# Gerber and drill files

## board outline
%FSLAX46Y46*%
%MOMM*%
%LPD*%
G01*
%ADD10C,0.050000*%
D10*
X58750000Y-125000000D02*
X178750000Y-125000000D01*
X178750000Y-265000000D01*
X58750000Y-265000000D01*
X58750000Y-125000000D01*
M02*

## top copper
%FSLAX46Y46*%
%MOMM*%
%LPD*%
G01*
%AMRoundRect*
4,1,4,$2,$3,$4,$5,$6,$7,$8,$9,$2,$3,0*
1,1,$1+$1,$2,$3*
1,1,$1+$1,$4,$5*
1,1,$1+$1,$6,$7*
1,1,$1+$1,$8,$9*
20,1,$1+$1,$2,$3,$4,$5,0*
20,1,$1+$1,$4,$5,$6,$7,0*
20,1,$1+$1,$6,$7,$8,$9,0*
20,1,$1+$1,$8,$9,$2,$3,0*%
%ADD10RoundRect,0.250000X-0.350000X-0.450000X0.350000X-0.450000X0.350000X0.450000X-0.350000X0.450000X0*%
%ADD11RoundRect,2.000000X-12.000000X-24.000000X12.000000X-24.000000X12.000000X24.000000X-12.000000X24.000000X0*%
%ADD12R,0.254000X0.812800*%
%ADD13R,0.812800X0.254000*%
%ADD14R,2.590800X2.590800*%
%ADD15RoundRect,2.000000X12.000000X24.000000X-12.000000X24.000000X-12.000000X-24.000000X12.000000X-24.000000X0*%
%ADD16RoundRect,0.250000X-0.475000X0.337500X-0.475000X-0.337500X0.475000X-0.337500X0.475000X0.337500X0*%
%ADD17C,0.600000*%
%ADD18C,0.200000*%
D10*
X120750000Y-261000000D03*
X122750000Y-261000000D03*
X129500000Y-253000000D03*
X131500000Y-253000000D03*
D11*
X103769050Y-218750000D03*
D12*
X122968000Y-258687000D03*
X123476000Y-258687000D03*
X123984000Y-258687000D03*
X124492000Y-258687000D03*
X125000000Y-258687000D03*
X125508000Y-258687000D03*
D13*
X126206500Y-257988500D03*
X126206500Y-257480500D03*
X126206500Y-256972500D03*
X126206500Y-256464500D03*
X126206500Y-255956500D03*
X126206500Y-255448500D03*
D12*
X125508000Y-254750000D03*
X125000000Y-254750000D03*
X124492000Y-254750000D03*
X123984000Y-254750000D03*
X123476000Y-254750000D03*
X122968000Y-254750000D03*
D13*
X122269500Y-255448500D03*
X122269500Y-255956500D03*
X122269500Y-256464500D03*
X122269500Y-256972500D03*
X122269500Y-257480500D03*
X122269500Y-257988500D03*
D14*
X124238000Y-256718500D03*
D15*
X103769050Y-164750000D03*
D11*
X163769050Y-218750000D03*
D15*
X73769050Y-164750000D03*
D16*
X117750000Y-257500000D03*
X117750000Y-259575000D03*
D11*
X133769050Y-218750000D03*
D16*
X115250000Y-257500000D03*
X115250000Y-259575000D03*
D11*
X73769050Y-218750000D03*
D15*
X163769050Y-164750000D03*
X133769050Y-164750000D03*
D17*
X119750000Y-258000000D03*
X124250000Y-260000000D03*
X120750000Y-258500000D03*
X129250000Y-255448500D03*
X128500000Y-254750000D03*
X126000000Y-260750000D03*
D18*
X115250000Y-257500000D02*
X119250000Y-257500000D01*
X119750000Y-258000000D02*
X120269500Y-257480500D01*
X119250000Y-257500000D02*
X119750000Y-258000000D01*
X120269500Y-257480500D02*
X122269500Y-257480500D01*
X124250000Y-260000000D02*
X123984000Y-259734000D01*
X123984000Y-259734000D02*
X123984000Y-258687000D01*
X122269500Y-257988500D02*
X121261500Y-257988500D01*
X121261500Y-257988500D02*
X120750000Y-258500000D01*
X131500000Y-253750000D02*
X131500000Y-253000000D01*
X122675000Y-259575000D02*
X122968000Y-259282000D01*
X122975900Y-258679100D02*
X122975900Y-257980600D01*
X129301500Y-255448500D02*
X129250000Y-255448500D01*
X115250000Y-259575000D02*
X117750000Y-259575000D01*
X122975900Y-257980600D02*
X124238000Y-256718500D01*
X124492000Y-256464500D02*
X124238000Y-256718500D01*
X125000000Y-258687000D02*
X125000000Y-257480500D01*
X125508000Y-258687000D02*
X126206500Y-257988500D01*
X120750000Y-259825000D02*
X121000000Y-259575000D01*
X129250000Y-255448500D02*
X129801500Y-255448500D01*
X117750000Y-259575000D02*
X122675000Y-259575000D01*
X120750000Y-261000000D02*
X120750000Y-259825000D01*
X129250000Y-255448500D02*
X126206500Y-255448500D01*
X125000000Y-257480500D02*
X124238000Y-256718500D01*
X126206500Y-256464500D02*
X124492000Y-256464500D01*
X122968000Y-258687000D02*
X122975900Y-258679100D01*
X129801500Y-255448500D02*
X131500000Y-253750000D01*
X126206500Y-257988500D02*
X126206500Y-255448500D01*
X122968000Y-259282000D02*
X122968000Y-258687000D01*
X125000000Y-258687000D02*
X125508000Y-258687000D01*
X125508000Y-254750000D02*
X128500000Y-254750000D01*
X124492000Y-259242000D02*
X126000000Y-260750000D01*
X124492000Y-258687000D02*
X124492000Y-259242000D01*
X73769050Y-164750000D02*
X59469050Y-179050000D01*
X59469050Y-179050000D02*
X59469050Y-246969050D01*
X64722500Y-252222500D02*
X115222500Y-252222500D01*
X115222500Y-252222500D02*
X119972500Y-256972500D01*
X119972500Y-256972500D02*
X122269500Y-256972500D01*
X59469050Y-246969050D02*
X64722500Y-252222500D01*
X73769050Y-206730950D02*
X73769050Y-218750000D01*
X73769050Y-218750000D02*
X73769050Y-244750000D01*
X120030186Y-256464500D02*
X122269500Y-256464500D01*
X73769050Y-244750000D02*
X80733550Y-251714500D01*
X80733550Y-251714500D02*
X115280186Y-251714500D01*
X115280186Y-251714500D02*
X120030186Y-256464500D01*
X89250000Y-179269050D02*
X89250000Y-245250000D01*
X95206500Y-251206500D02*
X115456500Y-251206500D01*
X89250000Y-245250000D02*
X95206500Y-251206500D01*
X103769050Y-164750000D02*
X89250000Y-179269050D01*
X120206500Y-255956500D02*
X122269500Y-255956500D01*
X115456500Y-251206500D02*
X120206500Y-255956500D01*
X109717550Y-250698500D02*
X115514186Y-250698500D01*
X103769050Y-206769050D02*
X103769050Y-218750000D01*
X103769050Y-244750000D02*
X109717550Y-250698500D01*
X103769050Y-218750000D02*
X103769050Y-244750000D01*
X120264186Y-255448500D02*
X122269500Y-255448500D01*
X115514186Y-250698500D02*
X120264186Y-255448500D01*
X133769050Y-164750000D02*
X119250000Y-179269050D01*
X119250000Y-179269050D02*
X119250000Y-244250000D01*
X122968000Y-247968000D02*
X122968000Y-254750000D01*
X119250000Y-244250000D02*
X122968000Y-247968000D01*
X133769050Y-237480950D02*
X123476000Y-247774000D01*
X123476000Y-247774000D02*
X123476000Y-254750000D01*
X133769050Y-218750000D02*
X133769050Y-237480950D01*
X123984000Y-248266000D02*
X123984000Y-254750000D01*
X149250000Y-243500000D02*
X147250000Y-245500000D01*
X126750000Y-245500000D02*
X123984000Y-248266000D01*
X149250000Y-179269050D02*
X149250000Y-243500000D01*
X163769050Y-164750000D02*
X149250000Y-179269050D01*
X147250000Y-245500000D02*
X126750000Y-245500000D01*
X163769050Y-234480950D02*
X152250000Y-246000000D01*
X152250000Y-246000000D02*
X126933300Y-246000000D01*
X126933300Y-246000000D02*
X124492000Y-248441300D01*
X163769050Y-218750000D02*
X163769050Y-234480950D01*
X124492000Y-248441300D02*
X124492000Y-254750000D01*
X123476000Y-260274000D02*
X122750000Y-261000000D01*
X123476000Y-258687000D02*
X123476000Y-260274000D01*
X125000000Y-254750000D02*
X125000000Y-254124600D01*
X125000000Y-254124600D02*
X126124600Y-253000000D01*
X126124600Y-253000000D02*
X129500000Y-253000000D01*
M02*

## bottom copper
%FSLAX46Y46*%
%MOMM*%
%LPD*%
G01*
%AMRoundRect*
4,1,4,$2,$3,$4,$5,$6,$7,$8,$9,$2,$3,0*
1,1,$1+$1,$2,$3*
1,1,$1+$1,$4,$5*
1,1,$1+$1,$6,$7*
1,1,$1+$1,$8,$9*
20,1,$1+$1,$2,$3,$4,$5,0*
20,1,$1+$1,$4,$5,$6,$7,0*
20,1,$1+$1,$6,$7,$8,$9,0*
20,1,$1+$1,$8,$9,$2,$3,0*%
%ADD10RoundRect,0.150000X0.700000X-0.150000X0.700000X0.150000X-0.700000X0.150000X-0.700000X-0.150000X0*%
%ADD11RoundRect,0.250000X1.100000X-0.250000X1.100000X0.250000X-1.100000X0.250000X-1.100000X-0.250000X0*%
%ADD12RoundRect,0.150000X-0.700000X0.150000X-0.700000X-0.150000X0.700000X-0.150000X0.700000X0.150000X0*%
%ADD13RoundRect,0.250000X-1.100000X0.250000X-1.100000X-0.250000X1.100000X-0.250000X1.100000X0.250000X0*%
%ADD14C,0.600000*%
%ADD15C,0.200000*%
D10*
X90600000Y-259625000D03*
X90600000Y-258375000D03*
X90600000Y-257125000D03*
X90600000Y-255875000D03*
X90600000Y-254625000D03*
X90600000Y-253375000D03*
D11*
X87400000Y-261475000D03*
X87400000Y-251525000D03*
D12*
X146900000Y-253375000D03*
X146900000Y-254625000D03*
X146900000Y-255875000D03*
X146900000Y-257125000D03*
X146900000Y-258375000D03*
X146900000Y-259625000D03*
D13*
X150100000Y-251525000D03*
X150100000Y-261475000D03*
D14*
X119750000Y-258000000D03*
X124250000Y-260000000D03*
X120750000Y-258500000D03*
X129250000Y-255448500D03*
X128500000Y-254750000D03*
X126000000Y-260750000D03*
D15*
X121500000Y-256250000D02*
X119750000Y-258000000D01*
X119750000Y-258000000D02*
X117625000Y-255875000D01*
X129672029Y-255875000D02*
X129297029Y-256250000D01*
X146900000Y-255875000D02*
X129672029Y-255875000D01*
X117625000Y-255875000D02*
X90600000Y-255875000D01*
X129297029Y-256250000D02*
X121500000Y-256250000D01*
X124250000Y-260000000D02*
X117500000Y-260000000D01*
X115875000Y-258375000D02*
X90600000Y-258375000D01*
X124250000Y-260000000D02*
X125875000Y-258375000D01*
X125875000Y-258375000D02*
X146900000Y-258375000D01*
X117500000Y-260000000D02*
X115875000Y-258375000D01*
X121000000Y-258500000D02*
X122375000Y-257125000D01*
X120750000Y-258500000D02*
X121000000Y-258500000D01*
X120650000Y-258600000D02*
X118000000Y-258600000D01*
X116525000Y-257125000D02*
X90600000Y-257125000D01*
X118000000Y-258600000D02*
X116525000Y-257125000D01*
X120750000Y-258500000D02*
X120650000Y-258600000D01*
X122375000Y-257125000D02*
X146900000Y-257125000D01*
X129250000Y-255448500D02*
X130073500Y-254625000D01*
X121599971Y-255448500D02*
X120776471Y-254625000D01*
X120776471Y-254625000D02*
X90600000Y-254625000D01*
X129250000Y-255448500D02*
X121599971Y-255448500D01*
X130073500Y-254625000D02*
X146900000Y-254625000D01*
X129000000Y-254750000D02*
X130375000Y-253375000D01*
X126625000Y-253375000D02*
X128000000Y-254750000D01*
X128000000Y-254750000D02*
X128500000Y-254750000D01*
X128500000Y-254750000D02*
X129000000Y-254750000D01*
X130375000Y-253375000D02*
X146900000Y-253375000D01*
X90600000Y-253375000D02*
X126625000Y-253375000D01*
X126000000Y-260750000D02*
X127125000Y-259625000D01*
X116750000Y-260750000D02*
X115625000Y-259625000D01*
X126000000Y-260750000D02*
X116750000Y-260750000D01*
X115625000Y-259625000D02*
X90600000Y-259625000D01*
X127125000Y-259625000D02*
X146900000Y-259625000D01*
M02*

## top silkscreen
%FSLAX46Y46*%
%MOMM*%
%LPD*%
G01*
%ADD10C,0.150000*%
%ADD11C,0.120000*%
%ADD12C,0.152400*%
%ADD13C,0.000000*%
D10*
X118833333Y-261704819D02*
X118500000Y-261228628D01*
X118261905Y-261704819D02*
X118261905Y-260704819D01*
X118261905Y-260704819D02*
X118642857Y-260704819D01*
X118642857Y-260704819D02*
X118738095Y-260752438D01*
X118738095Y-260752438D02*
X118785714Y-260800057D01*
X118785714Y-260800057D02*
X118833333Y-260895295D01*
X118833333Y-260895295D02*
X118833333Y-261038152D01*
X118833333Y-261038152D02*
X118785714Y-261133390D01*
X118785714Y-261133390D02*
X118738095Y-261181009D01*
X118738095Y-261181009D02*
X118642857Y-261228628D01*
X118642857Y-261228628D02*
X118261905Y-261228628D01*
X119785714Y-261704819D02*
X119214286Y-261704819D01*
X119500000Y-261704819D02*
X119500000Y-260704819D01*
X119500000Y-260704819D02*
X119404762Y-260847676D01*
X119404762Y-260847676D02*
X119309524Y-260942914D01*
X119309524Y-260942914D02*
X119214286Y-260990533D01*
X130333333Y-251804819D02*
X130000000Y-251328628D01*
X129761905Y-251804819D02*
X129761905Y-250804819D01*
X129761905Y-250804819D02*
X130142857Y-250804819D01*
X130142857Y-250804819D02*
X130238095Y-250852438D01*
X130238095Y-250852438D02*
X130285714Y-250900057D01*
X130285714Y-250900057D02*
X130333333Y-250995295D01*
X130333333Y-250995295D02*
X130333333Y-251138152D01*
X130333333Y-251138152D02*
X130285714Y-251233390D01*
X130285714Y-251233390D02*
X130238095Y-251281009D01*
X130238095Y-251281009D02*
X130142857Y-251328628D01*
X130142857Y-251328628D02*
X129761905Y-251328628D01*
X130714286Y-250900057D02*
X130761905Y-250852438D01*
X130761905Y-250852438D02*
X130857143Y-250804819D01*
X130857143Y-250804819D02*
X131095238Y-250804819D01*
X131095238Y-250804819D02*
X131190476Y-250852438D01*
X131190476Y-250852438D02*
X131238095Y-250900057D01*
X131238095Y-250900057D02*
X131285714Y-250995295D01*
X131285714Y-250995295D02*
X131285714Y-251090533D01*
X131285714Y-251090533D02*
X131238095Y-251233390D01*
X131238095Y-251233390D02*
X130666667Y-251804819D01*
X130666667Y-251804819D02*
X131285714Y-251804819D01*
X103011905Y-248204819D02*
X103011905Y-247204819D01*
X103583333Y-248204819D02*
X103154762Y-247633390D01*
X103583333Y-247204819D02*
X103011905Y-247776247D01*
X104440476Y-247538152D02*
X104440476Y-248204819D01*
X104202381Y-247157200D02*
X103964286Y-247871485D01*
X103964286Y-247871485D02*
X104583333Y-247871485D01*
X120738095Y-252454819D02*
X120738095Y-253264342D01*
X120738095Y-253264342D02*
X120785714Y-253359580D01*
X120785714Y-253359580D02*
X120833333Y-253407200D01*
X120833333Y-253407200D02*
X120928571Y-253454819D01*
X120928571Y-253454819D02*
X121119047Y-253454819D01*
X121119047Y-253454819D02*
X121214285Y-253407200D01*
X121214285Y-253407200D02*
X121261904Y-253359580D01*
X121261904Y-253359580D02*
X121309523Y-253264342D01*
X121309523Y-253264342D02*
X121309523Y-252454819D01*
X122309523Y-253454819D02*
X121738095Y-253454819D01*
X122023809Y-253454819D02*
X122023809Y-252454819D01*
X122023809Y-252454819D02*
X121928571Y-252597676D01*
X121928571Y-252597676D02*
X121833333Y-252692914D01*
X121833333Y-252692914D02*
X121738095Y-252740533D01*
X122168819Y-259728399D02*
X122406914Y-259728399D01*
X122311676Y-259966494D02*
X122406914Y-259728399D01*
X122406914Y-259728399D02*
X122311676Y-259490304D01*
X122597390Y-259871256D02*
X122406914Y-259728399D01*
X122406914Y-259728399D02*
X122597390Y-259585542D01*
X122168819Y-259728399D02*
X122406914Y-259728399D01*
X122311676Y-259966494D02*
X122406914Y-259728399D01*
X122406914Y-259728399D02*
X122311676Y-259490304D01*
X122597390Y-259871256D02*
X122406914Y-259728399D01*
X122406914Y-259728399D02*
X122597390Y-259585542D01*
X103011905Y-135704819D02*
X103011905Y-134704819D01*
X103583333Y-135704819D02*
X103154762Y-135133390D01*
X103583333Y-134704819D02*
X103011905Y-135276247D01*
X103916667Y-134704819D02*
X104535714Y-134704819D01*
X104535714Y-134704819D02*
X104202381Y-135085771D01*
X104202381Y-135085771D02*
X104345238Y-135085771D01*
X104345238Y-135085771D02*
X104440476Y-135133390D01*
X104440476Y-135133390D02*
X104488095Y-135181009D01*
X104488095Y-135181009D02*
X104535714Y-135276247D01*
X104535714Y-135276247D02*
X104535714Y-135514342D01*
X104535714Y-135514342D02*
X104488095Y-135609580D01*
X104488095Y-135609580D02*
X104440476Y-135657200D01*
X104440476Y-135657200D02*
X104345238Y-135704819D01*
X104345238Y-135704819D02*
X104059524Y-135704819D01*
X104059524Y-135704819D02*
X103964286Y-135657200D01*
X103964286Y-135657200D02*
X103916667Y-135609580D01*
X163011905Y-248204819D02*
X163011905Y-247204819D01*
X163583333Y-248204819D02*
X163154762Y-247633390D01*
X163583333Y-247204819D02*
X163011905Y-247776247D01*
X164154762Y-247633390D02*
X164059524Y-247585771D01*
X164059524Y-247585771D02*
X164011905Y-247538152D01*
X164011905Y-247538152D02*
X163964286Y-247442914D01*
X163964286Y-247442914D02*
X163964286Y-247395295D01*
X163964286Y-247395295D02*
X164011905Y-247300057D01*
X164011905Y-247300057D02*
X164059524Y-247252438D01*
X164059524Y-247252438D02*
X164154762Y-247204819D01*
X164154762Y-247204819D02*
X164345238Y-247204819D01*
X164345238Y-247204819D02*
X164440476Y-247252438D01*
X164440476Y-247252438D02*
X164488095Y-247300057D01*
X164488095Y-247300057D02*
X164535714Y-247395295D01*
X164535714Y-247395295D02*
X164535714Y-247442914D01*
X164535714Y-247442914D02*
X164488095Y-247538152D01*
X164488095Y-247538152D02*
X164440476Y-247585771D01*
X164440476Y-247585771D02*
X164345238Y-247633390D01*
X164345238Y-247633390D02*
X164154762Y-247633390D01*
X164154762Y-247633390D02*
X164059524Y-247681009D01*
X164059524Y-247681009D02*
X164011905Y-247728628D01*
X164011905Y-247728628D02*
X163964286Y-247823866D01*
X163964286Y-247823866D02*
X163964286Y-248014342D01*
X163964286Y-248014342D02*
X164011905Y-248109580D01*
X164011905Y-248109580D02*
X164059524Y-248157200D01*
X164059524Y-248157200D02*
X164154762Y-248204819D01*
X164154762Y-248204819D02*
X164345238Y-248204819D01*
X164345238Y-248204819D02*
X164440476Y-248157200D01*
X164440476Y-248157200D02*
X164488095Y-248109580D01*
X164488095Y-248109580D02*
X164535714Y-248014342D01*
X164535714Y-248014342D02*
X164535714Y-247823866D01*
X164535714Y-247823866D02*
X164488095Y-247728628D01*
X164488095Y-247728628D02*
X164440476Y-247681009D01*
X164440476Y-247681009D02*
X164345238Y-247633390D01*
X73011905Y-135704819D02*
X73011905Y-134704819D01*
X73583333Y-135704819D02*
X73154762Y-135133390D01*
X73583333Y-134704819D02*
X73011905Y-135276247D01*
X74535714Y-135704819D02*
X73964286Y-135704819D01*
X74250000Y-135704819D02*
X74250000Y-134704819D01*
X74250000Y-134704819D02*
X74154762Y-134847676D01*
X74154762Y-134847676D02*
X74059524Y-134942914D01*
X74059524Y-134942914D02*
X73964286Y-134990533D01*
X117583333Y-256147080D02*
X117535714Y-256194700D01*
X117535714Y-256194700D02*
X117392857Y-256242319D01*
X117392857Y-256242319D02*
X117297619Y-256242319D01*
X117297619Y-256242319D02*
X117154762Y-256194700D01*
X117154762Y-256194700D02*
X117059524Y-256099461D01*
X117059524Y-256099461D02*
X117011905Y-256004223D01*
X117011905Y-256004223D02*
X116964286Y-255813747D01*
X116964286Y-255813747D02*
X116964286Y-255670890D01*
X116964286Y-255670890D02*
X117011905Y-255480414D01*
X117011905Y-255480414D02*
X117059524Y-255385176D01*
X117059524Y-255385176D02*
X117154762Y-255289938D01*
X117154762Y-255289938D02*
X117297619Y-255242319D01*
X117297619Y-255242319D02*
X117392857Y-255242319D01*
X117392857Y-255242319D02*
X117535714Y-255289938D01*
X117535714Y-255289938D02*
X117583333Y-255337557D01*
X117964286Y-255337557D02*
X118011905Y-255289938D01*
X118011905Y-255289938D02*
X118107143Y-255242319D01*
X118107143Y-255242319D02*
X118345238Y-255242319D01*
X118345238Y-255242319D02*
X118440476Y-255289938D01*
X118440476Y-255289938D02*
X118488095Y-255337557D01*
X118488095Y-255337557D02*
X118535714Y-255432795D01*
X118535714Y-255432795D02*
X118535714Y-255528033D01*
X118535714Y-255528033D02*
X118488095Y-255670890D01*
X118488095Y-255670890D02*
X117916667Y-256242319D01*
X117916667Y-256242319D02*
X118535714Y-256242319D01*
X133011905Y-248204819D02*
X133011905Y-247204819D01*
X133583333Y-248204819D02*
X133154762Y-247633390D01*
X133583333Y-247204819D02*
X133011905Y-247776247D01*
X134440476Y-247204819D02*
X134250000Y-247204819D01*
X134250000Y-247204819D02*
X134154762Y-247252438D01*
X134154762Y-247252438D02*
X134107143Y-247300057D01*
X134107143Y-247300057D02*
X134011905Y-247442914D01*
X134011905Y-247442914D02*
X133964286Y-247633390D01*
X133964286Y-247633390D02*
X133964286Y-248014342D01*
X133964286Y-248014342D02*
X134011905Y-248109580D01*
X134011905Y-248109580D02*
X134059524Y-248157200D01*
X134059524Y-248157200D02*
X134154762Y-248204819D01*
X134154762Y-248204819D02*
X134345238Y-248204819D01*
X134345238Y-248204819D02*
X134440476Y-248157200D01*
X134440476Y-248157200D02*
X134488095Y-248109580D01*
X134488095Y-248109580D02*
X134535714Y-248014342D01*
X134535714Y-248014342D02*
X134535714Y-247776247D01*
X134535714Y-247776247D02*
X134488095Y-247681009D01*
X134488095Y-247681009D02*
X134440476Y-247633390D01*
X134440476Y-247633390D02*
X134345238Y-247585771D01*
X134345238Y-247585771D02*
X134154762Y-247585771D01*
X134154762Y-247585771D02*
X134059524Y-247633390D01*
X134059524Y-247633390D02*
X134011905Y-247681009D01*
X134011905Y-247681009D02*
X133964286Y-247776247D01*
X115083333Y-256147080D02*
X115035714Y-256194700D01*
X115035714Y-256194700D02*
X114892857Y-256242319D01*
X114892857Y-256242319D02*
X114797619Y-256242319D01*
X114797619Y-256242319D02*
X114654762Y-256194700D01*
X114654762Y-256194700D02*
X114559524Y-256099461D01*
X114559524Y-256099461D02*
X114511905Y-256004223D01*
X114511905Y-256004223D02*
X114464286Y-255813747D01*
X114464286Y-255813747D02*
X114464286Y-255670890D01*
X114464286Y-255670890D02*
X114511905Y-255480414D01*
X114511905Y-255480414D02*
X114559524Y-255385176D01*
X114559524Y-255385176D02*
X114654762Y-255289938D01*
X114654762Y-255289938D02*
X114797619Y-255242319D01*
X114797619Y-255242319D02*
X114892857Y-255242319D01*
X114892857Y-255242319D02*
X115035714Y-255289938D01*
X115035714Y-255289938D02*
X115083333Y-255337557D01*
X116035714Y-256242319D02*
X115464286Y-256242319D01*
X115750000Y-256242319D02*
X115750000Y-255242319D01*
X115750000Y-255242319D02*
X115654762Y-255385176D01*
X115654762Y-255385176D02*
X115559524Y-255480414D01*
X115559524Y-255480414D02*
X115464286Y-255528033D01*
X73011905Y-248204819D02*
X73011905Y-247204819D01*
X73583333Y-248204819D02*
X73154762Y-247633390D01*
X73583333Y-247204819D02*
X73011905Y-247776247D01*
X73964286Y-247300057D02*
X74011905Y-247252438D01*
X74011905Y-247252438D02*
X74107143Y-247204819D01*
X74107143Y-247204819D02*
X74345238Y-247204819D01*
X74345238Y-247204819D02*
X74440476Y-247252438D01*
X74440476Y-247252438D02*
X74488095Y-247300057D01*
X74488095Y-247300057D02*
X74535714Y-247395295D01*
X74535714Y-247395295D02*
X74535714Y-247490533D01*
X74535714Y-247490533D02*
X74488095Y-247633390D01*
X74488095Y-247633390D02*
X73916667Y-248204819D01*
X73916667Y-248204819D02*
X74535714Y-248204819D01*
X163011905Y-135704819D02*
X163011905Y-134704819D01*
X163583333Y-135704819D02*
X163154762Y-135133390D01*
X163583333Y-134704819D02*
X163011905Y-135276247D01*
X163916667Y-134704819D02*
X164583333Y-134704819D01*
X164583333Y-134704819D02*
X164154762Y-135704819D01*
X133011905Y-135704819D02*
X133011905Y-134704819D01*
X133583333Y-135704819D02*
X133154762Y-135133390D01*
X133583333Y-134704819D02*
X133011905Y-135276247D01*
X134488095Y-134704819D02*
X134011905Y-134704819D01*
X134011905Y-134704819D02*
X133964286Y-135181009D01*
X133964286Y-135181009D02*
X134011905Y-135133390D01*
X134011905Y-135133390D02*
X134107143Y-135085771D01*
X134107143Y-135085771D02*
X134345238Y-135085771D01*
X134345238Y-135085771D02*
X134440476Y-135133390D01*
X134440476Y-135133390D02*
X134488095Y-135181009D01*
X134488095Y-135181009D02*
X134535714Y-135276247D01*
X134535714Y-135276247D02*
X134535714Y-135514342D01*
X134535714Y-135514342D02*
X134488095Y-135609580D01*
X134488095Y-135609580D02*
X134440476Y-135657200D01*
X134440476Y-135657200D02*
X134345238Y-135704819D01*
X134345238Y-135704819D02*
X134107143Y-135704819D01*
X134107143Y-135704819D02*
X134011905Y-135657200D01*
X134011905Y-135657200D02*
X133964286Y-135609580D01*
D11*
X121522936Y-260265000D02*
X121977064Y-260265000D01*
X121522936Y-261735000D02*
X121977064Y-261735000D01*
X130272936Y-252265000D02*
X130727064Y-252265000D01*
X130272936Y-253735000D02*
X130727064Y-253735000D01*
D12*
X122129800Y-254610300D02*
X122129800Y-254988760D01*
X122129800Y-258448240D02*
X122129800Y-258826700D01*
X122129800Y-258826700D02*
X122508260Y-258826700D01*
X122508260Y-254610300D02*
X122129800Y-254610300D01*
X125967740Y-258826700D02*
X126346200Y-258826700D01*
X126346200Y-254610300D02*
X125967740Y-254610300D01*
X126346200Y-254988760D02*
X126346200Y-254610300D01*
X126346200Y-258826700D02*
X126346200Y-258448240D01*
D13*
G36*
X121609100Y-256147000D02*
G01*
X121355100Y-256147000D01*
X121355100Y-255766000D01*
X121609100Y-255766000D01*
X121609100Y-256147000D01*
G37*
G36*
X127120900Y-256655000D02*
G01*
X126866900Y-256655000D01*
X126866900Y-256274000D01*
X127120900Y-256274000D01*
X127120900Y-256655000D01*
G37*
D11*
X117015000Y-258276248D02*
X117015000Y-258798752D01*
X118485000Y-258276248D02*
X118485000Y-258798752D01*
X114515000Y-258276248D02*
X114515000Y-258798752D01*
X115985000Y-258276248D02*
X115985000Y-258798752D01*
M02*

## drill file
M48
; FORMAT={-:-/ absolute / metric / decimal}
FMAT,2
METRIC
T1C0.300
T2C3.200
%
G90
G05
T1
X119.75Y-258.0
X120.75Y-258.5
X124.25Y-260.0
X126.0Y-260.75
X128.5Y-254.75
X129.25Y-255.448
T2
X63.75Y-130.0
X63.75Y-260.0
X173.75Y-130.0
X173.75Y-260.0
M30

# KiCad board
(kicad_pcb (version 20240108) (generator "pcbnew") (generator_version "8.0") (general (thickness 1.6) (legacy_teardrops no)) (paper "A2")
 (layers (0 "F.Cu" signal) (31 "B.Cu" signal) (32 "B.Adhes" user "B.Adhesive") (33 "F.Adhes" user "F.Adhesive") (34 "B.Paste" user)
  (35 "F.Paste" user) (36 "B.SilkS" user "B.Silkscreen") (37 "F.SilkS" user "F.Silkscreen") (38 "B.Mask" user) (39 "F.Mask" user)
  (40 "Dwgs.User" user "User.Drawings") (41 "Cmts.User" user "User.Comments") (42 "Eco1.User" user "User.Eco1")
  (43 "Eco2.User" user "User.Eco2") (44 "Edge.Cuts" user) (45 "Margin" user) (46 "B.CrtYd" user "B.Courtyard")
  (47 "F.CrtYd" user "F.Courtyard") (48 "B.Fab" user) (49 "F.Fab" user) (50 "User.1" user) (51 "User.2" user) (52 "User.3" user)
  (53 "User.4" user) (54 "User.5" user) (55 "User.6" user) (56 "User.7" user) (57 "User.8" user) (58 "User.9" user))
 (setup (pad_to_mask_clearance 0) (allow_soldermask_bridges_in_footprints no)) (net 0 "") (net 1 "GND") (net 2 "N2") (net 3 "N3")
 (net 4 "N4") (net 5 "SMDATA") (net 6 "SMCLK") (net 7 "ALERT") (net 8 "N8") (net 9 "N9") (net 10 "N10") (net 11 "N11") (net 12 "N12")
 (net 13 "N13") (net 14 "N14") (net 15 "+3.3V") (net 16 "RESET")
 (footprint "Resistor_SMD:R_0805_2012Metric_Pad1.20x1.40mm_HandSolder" (layer "F.Cu") (at 121.75 261)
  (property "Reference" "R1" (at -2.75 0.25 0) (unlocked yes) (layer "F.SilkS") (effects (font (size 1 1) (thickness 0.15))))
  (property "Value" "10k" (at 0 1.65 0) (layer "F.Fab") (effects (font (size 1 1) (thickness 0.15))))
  (fp_line (start -0.227064 -0.735) (end 0.227064 -0.735) (stroke (width 0.12) (type solid)) (layer "F.SilkS"))
  (fp_line (start -0.227064 0.735) (end 0.227064 0.735) (stroke (width 0.12) (type solid)) (layer "F.SilkS"))
  (pad "1" smd roundrect (at -1 0) (size 1.2 1.4) (layers "F.Cu" "F.Paste" "F.Mask") (roundrect_rratio 0.208333) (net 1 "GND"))
  (pad "2" smd roundrect (at 1 0) (size 1.2 1.4) (layers "F.Cu" "F.Paste" "F.Mask") (roundrect_rratio 0.208333) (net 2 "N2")))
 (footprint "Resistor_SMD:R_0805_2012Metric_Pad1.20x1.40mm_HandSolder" (layer "F.Cu") (at 130.5 253)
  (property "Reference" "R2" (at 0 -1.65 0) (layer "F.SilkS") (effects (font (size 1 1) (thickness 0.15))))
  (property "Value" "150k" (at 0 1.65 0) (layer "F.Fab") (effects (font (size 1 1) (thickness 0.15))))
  (fp_line (start -0.227064 -0.735) (end 0.227064 -0.735) (stroke (width 0.12) (type solid)) (layer "F.SilkS"))
  (fp_line (start -0.227064 0.735) (end 0.227064 0.735) (stroke (width 0.12) (type solid)) (layer "F.SilkS"))
  (pad "1" smd roundrect (at -1 0) (size 1.2 1.4) (layers "F.Cu" "F.Paste" "F.Mask") (roundrect_rratio 0.208333) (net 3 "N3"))
  (pad "2" smd roundrect (at 1 0) (size 1.2 1.4) (layers "F.Cu" "F.Paste" "F.Mask") (roundrect_rratio 0.208333) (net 1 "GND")))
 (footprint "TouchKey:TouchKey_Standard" (layer "F.Cu") (at 103.76905 218.75)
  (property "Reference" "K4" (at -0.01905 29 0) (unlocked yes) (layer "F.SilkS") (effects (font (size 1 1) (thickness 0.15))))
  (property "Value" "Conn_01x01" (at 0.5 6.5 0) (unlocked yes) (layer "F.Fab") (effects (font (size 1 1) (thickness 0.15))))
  (pad "1" smd roundrect (at 0 0) (size 28 52) (layers "F.Cu") (roundrect_rratio 0.07142857143) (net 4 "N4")))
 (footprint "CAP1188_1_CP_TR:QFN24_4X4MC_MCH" (layer "F.Cu") (at 124.238 256.7185 90)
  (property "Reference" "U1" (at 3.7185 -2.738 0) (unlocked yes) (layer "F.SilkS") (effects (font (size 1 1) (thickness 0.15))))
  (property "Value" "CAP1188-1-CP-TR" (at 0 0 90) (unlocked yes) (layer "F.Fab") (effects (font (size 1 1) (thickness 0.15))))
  (fp_line (start 2.1082 -2.1082) (end 1.72974 -2.1082) (stroke (width 0.1524) (type solid)) (layer "F.SilkS"))
  (fp_line (start -1.72974 -2.1082) (end -2.1082 -2.1082) (stroke (width 0.1524) (type solid)) (layer "F.SilkS"))
  (fp_line (start -2.1082 -2.1082) (end -2.1082 -1.72974) (stroke (width 0.1524) (type solid)) (layer "F.SilkS"))
  (fp_line (start 2.1082 -1.72974) (end 2.1082 -2.1082) (stroke (width 0.1524) (type solid)) (layer "F.SilkS"))
  (fp_line (start -2.1082 1.72974) (end -2.1082 2.1082) (stroke (width 0.1524) (type solid)) (layer "F.SilkS"))
  (fp_line (start 2.1082 2.1082) (end 2.1082 1.72974) (stroke (width 0.1524) (type solid)) (layer "F.SilkS"))
  (fp_line (start 1.72974 2.1082) (end 2.1082 2.1082) (stroke (width 0.1524) (type solid)) (layer "F.SilkS"))
  (fp_line (start -2.1082 2.1082) (end -1.72974 2.1082) (stroke (width 0.1524) (type solid)) (layer "F.SilkS"))
  (fp_poly
   (pts (xy 0.5715 -2.6289) (xy 0.5715 -2.8829) (xy 0.9525 -2.8829) (xy 0.9525 -2.6289)) (stroke (width 0) (type solid)) (fill solid)
   (layer "F.SilkS"))
  (fp_poly
   (pts (xy 0.0635 2.6289) (xy 0.0635 2.8829) (xy 0.4445 2.8829) (xy 0.4445 2.6289)) (stroke (width 0) (type solid)) (fill solid)
   (layer "F.SilkS"))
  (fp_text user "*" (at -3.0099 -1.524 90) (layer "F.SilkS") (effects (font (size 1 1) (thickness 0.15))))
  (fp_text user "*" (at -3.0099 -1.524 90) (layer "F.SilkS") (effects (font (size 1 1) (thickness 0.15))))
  (pad "1" smd rect (at -1.9685 -1.27 180) (size 0.254 0.8128) (layers "F.Cu" "F.Paste" "F.Mask") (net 1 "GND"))
  (pad "2" smd rect (at -1.9685 -0.762 180) (size 0.254 0.8128) (layers "F.Cu" "F.Paste" "F.Mask") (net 2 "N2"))
  (pad "3" smd rect (at -1.9685 -0.254 180) (size 0.254 0.8128) (layers "F.Cu" "F.Paste" "F.Mask") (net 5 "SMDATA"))
  (pad "4" smd rect (at -1.9685 0.254 180) (size 0.254 0.8128) (layers "F.Cu" "F.Paste" "F.Mask") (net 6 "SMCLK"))
  (pad "5" smd rect (at -1.9685 0.762 180) (size 0.254 0.8128) (layers "F.Cu" "F.Paste" "F.Mask") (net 1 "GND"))
  (pad "6" smd rect (at -1.9685 1.27 180) (size 0.254 0.8128) (layers "F.Cu" "F.Paste" "F.Mask") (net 1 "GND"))
  (pad "7" smd rect (at -1.27 1.9685 90) (size 0.254 0.8128) (layers "F.Cu" "F.Paste" "F.Mask") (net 1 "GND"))
  (pad "8" smd rect (at -0.762 1.9685 90) (size 0.254 0.8128) (layers "F.Cu" "F.Paste" "F.Mask") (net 1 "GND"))
  (pad "9" smd rect (at -0.254 1.9685 90) (size 0.254 0.8128) (layers "F.Cu" "F.Paste" "F.Mask") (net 1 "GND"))
  (pad "10" smd rect (at 0.254 1.9685 90) (size 0.254 0.8128) (layers "F.Cu" "F.Paste" "F.Mask") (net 1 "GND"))
  (pad "11" smd rect (at 0.762 1.9685 90) (size 0.254 0.8128) (layers "F.Cu" "F.Paste" "F.Mask") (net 1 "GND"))
  (pad "12" smd rect (at 1.27 1.9685 90) (size 0.254 0.8128) (layers "F.Cu" "F.Paste" "F.Mask") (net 1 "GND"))
  (pad "13" smd rect (at 1.9685 1.27 180) (size 0.254 0.8128) (layers "F.Cu" "F.Paste" "F.Mask") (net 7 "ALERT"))
  (pad "14" smd rect (at 1.9685 0.762 180) (size 0.254 0.8128) (layers "F.Cu" "F.Paste" "F.Mask") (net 3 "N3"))
  (pad "15" smd rect (at 1.9685 0.254 180) (size 0.254 0.8128) (layers "F.Cu" "F.Paste" "F.Mask") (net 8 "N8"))
  (pad "16" smd rect (at 1.9685 -0.254 180) (size 0.254 0.8128) (layers "F.Cu" "F.Paste" "F.Mask") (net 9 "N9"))
  (pad "17" smd rect (at 1.9685 -0.762 180) (size 0.254 0.8128) (layers "F.Cu" "F.Paste" "F.Mask") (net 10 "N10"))
  (pad "18" smd rect (at 1.9685 -1.27 180) (size 0.254 0.8128) (layers "F.Cu" "F.Paste" "F.Mask") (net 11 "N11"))
  (pad "19" smd rect (at 1.27 -1.9685 90) (size 0.254 0.8128) (layers "F.Cu" "F.Paste" "F.Mask") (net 4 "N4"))
  (pad "20" smd rect (at 0.762 -1.9685 90) (size 0.254 0.8128) (layers "F.Cu" "F.Paste" "F.Mask") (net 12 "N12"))
  (pad "21" smd rect (at 0.254 -1.9685 90) (size 0.254 0.8128) (layers "F.Cu" "F.Paste" "F.Mask") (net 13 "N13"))
  (pad "22" smd rect (at -0.254 -1.9685 90) (size 0.254 0.8128) (layers "F.Cu" "F.Paste" "F.Mask") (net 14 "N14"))
  (pad "23" smd rect (at -0.762 -1.9685 90) (size 0.254 0.8128) (layers "F.Cu" "F.Paste" "F.Mask") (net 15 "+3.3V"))
  (pad "24" smd rect (at -1.27 -1.9685 90) (size 0.254 0.8128) (layers "F.Cu" "F.Paste" "F.Mask") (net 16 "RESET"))
  (pad "25" smd rect (at 0 0 90) (size 2.5908 2.5908) (layers "F.Cu" "F.Paste" "F.Mask") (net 1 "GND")))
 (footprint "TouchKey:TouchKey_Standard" (layer "F.Cu") (at 103.76905 164.75 180)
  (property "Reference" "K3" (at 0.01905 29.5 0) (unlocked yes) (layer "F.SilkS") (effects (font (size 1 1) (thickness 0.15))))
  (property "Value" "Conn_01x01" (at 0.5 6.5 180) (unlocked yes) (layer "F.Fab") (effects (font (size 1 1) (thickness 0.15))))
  (pad "1" smd roundrect (at 0 0 180) (size 28 52) (layers "F.Cu") (roundrect_rratio 0.07142857143) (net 12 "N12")))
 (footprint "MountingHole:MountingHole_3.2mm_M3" (layer "F.Cu") (at 173.75 130)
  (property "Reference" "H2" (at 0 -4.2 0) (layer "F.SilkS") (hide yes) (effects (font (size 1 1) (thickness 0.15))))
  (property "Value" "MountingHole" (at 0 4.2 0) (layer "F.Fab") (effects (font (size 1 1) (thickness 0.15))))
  (pad "" np_thru_hole circle (at 0 0) (size 3.2 3.2) (drill 3.2) (layers "*.Cu" "*.Mask")))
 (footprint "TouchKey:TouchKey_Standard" (layer "F.Cu") (at 163.76905 218.75)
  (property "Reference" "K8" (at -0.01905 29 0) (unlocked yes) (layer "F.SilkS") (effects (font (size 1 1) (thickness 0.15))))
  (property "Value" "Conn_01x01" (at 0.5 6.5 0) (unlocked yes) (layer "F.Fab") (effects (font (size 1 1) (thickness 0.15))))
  (pad "1" smd roundrect (at 0 0) (size 28 52) (layers "F.Cu") (roundrect_rratio 0.07142857143) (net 8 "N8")))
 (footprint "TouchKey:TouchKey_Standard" (layer "F.Cu") (at 73.76905 164.75 180)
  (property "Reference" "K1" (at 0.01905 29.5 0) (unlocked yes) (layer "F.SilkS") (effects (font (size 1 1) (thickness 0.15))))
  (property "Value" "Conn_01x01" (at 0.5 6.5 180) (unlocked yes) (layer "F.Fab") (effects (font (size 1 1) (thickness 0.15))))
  (pad "1" smd roundrect (at 0 0 180) (size 28 52) (layers "F.Cu") (roundrect_rratio 0.07142857143) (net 14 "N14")))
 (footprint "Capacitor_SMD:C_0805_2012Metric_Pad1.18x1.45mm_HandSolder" (layer "F.Cu") (at 117.75 258.5375 -90)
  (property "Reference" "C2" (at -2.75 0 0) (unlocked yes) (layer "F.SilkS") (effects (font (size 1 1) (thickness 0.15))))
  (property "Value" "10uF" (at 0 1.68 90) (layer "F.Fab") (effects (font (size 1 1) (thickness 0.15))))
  (fp_line (start -0.261252 0.735) (end 0.261252 0.735) (stroke (width 0.12) (type solid)) (layer "F.SilkS"))
  (fp_line (start -0.261252 -0.735) (end 0.261252 -0.735) (stroke (width 0.12) (type solid)) (layer "F.SilkS"))
  (pad "1" smd roundrect (at -1.0375 0 270) (size 1.175 1.45) (layers "F.Cu" "F.Paste" "F.Mask") (roundrect_rratio 0.212766)
   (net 15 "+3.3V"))
  (pad "2" smd roundrect (at 1.0375 0 270) (size 1.175 1.45) (layers "F.Cu" "F.Paste" "F.Mask") (roundrect_rratio 0.212766) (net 1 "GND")))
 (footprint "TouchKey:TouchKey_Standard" (layer "F.Cu") (at 133.76905 218.75)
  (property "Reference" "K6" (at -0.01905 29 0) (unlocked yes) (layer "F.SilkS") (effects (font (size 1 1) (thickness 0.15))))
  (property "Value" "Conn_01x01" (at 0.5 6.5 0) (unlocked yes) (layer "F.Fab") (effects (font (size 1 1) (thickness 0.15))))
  (pad "1" smd roundrect (at 0 0) (size 28 52) (layers "F.Cu") (roundrect_rratio 0.07142857143) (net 10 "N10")))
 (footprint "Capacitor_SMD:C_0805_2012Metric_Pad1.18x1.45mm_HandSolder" (layer "F.Cu") (at 115.25 258.5375 -90)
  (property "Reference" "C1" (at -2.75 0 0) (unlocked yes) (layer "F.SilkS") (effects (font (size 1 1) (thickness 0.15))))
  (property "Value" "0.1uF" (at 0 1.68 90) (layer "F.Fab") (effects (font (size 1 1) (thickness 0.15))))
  (fp_line (start -0.261252 0.735) (end 0.261252 0.735) (stroke (width 0.12) (type solid)) (layer "F.SilkS"))
  (fp_line (start -0.261252 -0.735) (end 0.261252 -0.735) (stroke (width 0.12) (type solid)) (layer "F.SilkS"))
  (pad "1" smd roundrect (at -1.0375 0 270) (size 1.175 1.45) (layers "F.Cu" "F.Paste" "F.Mask") (roundrect_rratio 0.212766)
   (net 15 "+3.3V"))
  (pad "2" smd roundrect (at 1.0375 0 270) (size 1.175 1.45) (layers "F.Cu" "F.Paste" "F.Mask") (roundrect_rratio 0.212766) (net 1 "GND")))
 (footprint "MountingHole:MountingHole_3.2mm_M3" (layer "F.Cu") (at 63.75 260)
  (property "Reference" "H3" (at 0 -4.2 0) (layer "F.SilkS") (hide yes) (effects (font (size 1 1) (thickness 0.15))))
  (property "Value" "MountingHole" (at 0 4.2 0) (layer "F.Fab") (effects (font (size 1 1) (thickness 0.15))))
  (pad "" np_thru_hole circle (at 0 0) (size 3.2 3.2) (drill 3.2) (layers "*.Cu" "*.Mask")))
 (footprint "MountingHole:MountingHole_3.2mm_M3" (layer "F.Cu") (at 63.75 130)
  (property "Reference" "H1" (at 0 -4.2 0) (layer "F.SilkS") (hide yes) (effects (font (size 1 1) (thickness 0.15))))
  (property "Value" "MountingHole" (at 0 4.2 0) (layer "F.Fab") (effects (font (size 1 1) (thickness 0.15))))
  (pad "" np_thru_hole circle (at 0 0) (size 3.2 3.2) (drill 3.2) (layers "*.Cu" "*.Mask")))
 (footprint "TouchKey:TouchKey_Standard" (layer "F.Cu") (at 73.76905 218.75)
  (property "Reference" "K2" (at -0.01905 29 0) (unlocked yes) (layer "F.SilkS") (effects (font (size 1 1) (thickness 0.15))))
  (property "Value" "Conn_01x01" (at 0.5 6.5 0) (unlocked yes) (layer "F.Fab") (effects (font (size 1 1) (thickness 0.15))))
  (pad "1" smd roundrect (at 0 0) (size 28 52) (layers "F.Cu") (roundrect_rratio 0.07142857143) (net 13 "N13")))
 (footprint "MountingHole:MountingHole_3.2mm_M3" (layer "F.Cu") (at 173.75 260)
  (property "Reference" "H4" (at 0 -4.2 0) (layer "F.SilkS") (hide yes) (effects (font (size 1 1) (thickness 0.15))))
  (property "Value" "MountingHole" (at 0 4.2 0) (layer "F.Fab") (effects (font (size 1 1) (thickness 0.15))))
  (pad "" np_thru_hole circle (at 0 0) (size 3.2 3.2) (drill 3.2) (layers "*.Cu" "*.Mask")))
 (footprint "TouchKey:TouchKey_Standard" (layer "F.Cu") (at 163.76905 164.75 180)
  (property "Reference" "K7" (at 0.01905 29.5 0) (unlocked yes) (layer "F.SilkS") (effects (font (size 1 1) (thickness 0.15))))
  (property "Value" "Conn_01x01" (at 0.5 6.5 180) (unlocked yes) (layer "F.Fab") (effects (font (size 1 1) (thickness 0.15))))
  (pad "1" smd roundrect (at 0 0 180) (size 28 52) (layers "F.Cu") (roundrect_rratio 0.07142857143) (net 9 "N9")))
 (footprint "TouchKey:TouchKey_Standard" (layer "F.Cu") (at 133.76905 164.75 180)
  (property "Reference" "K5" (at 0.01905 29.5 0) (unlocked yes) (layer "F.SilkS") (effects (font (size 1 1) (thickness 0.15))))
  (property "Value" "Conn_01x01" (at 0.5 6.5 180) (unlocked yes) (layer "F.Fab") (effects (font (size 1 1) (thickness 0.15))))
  (pad "1" smd roundrect (at 0 0 180) (size 28 52) (layers "F.Cu") (roundrect_rratio 0.07142857143) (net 11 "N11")))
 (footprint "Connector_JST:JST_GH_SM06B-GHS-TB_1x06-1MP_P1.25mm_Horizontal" (layer "B.Cu") (at 88.75 256.5 90)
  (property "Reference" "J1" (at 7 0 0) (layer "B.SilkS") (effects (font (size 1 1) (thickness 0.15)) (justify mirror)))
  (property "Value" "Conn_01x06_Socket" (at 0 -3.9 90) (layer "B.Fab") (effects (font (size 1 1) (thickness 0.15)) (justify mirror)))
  (pad "1" smd roundrect (at -3.125 1.85 90) (size 0.6 1.7) (layers "B.Cu" "B.Paste" "B.Mask") (roundrect_rratio 0.25) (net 6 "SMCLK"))
  (pad "2" smd roundrect (at -1.875 1.85 90) (size 0.6 1.7) (layers "B.Cu" "B.Paste" "B.Mask") (roundrect_rratio 0.25) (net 5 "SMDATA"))
  (pad "3" smd roundrect (at -0.625 1.85 90) (size 0.6 1.7) (layers "B.Cu" "B.Paste" "B.Mask") (roundrect_rratio 0.25) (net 16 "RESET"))
  (pad "4" smd roundrect (at 0.625 1.85 90) (size 0.6 1.7) (layers "B.Cu" "B.Paste" "B.Mask") (roundrect_rratio 0.25) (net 15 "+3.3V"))
  (pad "5" smd roundrect (at 1.875 1.85 90) (size 0.6 1.7) (layers "B.Cu" "B.Paste" "B.Mask") (roundrect_rratio 0.25) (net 1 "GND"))
  (pad "6" smd roundrect (at 3.125 1.85 90) (size 0.6 1.7) (layers "B.Cu" "B.Paste" "B.Mask") (roundrect_rratio 0.25) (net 7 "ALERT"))
  (pad "MP" smd roundrect (at -4.975 -1.35 90) (size 1 2.7) (layers "B.Cu" "B.Paste" "B.Mask") (roundrect_rratio 0.25))
  (pad "MP" smd roundrect (at 4.975 -1.35 90) (size 1 2.7) (layers "B.Cu" "B.Paste" "B.Mask") (roundrect_rratio 0.25)))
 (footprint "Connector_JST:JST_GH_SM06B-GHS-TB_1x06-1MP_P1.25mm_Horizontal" (layer "B.Cu") (at 148.75 256.5 -90)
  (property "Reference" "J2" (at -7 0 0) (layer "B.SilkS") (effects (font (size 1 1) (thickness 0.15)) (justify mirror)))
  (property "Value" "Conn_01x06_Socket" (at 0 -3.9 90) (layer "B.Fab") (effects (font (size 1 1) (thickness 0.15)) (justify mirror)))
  (pad "1" smd roundrect (at -3.125 1.85 270) (size 0.6 1.7) (layers "B.Cu" "B.Paste" "B.Mask") (roundrect_rratio 0.25) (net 7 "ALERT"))
  (pad "2" smd roundrect (at -1.875 1.85 270) (size 0.6 1.7) (layers "B.Cu" "B.Paste" "B.Mask") (roundrect_rratio 0.25) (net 1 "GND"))
  (pad "3" smd roundrect (at -0.625 1.85 270) (size 0.6 1.7) (layers "B.Cu" "B.Paste" "B.Mask") (roundrect_rratio 0.25) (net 15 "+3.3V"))
  (pad "4" smd roundrect (at 0.625 1.85 270) (size 0.6 1.7) (layers "B.Cu" "B.Paste" "B.Mask") (roundrect_rratio 0.25) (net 16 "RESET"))
  (pad "5" smd roundrect (at 1.875 1.85 270) (size 0.6 1.7) (layers "B.Cu" "B.Paste" "B.Mask") (roundrect_rratio 0.25) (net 5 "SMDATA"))
  (pad "6" smd roundrect (at 3.125 1.85 270) (size 0.6 1.7) (layers "B.Cu" "B.Paste" "B.Mask") (roundrect_rratio 0.25) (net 6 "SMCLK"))
  (pad "MP" smd roundrect (at -4.975 -1.35 270) (size 1 2.7) (layers "B.Cu" "B.Paste" "B.Mask") (roundrect_rratio 0.25))
  (pad "MP" smd roundrect (at 4.975 -1.35 270) (size 1 2.7) (layers "B.Cu" "B.Paste" "B.Mask") (roundrect_rratio 0.25)))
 (gr_rect (start 58.75 125) (end 178.75 265) (stroke (width 0.05) (type default)) (fill none) (layer "Edge.Cuts"))
 (segment (start 115.25 257.5) (end 119.25 257.5) (width 0.2) (layer "F.Cu") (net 15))
 (segment (start 119.75 258) (end 120.2695 257.4805) (width 0.2) (layer "F.Cu") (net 15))
 (segment (start 119.25 257.5) (end 119.75 258) (width 0.2) (layer "F.Cu") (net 15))
 (segment (start 120.2695 257.4805) (end 122.2695 257.4805) (width 0.2) (layer "F.Cu") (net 15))
 (via (at 119.75 258) (size 0.6) (drill 0.3) (layers "F.Cu" "B.Cu") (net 15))
 (segment (start 121.5 256.25) (end 119.75 258) (width 0.2) (layer "B.Cu") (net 15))
 (segment (start 119.75 258) (end 117.625 255.875) (width 0.2) (layer "B.Cu") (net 15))
 (segment (start 129.672029 255.875) (end 129.297029 256.25) (width 0.2) (layer "B.Cu") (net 15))
 (segment (start 146.9 255.875) (end 129.672029 255.875) (width 0.2) (layer "B.Cu") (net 15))
 (segment (start 117.625 255.875) (end 90.6 255.875) (width 0.2) (layer "B.Cu") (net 15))
 (segment (start 129.297029 256.25) (end 121.5 256.25) (width 0.2) (layer "B.Cu") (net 15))
 (segment (start 124.25 260) (end 123.984 259.734) (width 0.2) (layer "F.Cu") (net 5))
 (segment (start 123.984 259.734) (end 123.984 258.687) (width 0.2) (layer "F.Cu") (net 5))
 (via (at 124.25 260) (size 0.6) (drill 0.3) (layers "F.Cu" "B.Cu") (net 5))
 (segment (start 124.25 260) (end 117.5 260) (width 0.2) (layer "B.Cu") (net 5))
 (segment (start 115.875 258.375) (end 90.6 258.375) (width 0.2) (layer "B.Cu") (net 5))
 (segment (start 124.25 260) (end 125.875 258.375) (width 0.2) (layer "B.Cu") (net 5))
 (segment (start 125.875 258.375) (end 146.9 258.375) (width 0.2) (layer "B.Cu") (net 5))
 (segment (start 117.5 260) (end 115.875 258.375) (width 0.2) (layer "B.Cu") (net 5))
 (segment (start 122.2695 257.9885) (end 121.2615 257.9885) (width 0.2) (layer "F.Cu") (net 16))
 (segment (start 121.2615 257.9885) (end 120.75 258.5) (width 0.2) (layer "F.Cu") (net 16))
 (via (at 120.75 258.5) (size 0.6) (drill 0.3) (layers "F.Cu" "B.Cu") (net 16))
 (segment (start 121 258.5) (end 122.375 257.125) (width 0.2) (layer "B.Cu") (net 16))
 (segment (start 120.75 258.5) (end 121 258.5) (width 0.2) (layer "B.Cu") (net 16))
 (segment (start 120.65 258.6) (end 118 258.6) (width 0.2) (layer "B.Cu") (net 16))
 (segment (start 116.525 257.125) (end 90.6 257.125) (width 0.2) (layer "B.Cu") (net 16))
 (segment (start 118 258.6) (end 116.525 257.125) (width 0.2) (layer "B.Cu") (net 16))
 (segment (start 120.75 258.5) (end 120.65 258.6) (width 0.2) (layer "B.Cu") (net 16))
 (segment (start 122.375 257.125) (end 146.9 257.125) (width 0.2) (layer "B.Cu") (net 16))
 (segment (start 131.5 253.75) (end 131.5 253) (width 0.2) (layer "F.Cu") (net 1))
 (segment (start 122.675 259.575) (end 122.968 259.282) (width 0.2) (layer "F.Cu") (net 1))
 (segment (start 122.9759 258.6791) (end 122.9759 257.9806) (width 0.2) (layer "F.Cu") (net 1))
 (segment (start 129.3015 255.4485) (end 129.25 255.4485) (width 0.2) (layer "F.Cu") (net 1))
 (segment (start 115.25 259.575) (end 117.75 259.575) (width 0.2) (layer "F.Cu") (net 1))
 (segment (start 122.9759 257.9806) (end 124.238 256.7185) (width 0.2) (layer "F.Cu") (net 1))
 (segment (start 124.492 256.4645) (end 124.238 256.7185) (width 0.2) (layer "F.Cu") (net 1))
 (segment (start 125 258.687) (end 125 257.4805) (width 0.2) (layer "F.Cu") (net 1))
 (segment (start 125.508 258.687) (end 126.2065 257.9885) (width 0.2) (layer "F.Cu") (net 1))
 (segment (start 120.75 259.825) (end 121 259.575) (width 0.2) (layer "F.Cu") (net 1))
 (segment (start 129.25 255.4485) (end 129.8015 255.4485) (width 0.2) (layer "F.Cu") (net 1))
 (segment (start 117.75 259.575) (end 122.675 259.575) (width 0.2) (layer "F.Cu") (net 1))
 (segment (start 120.75 261) (end 120.75 259.825) (width 0.2) (layer "F.Cu") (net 1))
 (segment (start 129.25 255.4485) (end 126.2065 255.4485) (width 0.2) (layer "F.Cu") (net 1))
 (segment (start 125 257.4805) (end 124.238 256.7185) (width 0.2) (layer "F.Cu") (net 1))
 (segment (start 126.2065 256.4645) (end 124.492 256.4645) (width 0.2) (layer "F.Cu") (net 1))
 (segment (start 122.968 258.687) (end 122.9759 258.6791) (width 0.2) (layer "F.Cu") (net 1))
 (segment (start 129.8015 255.4485) (end 131.5 253.75) (width 0.2) (layer "F.Cu") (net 1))
 (segment (start 126.2065 257.9885) (end 126.2065 255.4485) (width 0.2) (layer "F.Cu") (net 1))
 (segment (start 122.968 259.282) (end 122.968 258.687) (width 0.2) (layer "F.Cu") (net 1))
 (segment (start 125 258.687) (end 125.508 258.687) (width 0.2) (layer "F.Cu") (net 1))
 (via (at 129.25 255.4485) (size 0.6) (drill 0.3) (layers "F.Cu" "B.Cu") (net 1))
 (segment (start 129.25 255.4485) (end 130.0735 254.625) (width 0.2) (layer "B.Cu") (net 1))
 (segment (start 121.599971 255.4485) (end 120.776471 254.625) (width 0.2) (layer "B.Cu") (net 1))
 (segment (start 120.776471 254.625) (end 90.6 254.625) (width 0.2) (layer "B.Cu") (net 1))
 (segment (start 129.25 255.4485) (end 121.599971 255.4485) (width 0.2) (layer "B.Cu") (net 1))
 (segment (start 130.0735 254.625) (end 146.9 254.625) (width 0.2) (layer "B.Cu") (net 1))
 (segment (start 125.508 254.75) (end 128.5 254.75) (width 0.2) (layer "F.Cu") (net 7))
 (via (at 128.5 254.75) (size 0.6) (drill 0.3) (layers "F.Cu" "B.Cu") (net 7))
 (segment (start 129 254.75) (end 130.375 253.375) (width 0.2) (layer "B.Cu") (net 7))
 (segment (start 126.625 253.375) (end 128 254.75) (width 0.2) (layer "B.Cu") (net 7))
 (segment (start 128 254.75) (end 128.5 254.75) (width 0.2) (layer "B.Cu") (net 7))
 (segment (start 128.5 254.75) (end 129 254.75) (width 0.2) (layer "B.Cu") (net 7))
 (segment (start 130.375 253.375) (end 146.9 253.375) (width 0.2) (layer "B.Cu") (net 7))
 (segment (start 90.6 253.375) (end 126.625 253.375) (width 0.2) (layer "B.Cu") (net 7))
 (segment (start 124.492 259.242) (end 126 260.75) (width 0.2) (layer "F.Cu") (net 6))
 (segment (start 124.492 258.687) (end 124.492 259.242) (width 0.2) (layer "F.Cu") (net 6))
 (via (at 126 260.75) (size 0.6) (drill 0.3) (layers "F.Cu" "B.Cu") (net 6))
 (segment (start 126 260.75) (end 127.125 259.625) (width 0.2) (layer "B.Cu") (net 6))
 (segment (start 116.75 260.75) (end 115.625 259.625) (width 0.2) (layer "B.Cu") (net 6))
 (segment (start 126 260.75) (end 116.75 260.75) (width 0.2) (layer "B.Cu") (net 6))
 (segment (start 115.625 259.625) (end 90.6 259.625) (width 0.2) (layer "B.Cu") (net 6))
 (segment (start 127.125 259.625) (end 146.9 259.625) (width 0.2) (layer "B.Cu") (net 6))
 (segment (start 73.76905 164.75) (end 59.46905 179.05) (width 0.2) (layer "F.Cu") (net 14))
 (segment (start 59.46905 179.05) (end 59.46905 246.96905) (width 0.2) (layer "F.Cu") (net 14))
 (segment (start 64.7225 252.2225) (end 115.2225 252.2225) (width 0.2) (layer "F.Cu") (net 14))
 (segment (start 115.2225 252.2225) (end 119.9725 256.9725) (width 0.2) (layer "F.Cu") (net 14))
 (segment (start 119.9725 256.9725) (end 122.2695 256.9725) (width 0.2) (layer "F.Cu") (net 14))
 (segment (start 59.46905 246.96905) (end 64.7225 252.2225) (width 0.2) (layer "F.Cu") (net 14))
 (segment (start 73.76905 206.73095) (end 73.76905 218.75) (width 0.2) (layer "F.Cu") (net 13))
 (segment (start 73.76905 218.75) (end 73.76905 244.75) (width 0.2) (layer "F.Cu") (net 13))
 (segment (start 120.030186 256.4645) (end 122.2695 256.4645) (width 0.2) (layer "F.Cu") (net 13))
 (segment (start 73.76905 244.75) (end 80.73355 251.7145) (width 0.2) (layer "F.Cu") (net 13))
 (segment (start 80.73355 251.7145) (end 115.280186 251.7145) (width 0.2) (layer "F.Cu") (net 13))
 (segment (start 115.280186 251.7145) (end 120.030186 256.4645) (width 0.2) (layer "F.Cu") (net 13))
 (segment (start 89.25 179.26905) (end 89.25 245.25) (width 0.2) (layer "F.Cu") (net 12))
 (segment (start 95.2065 251.2065) (end 115.4565 251.2065) (width 0.2) (layer "F.Cu") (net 12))
 (segment (start 89.25 245.25) (end 95.2065 251.2065) (width 0.2) (layer "F.Cu") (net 12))
 (segment (start 103.76905 164.75) (end 89.25 179.26905) (width 0.2) (layer "F.Cu") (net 12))
 (segment (start 120.2065 255.9565) (end 122.2695 255.9565) (width 0.2) (layer "F.Cu") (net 12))
 (segment (start 115.4565 251.2065) (end 120.2065 255.9565) (width 0.2) (layer "F.Cu") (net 12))
 (segment (start 109.71755 250.6985) (end 115.514186 250.6985) (width 0.2) (layer "F.Cu") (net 4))
 (segment (start 103.76905 206.76905) (end 103.76905 218.75) (width 0.2) (layer "F.Cu") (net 4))
 (segment (start 103.76905 244.75) (end 109.71755 250.6985) (width 0.2) (layer "F.Cu") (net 4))
 (segment (start 103.76905 218.75) (end 103.76905 244.75) (width 0.2) (layer "F.Cu") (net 4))
 (segment (start 120.264186 255.4485) (end 122.2695 255.4485) (width 0.2) (layer "F.Cu") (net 4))
 (segment (start 115.514186 250.6985) (end 120.264186 255.4485) (width 0.2) (layer "F.Cu") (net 4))
 (segment (start 133.76905 164.75) (end 119.25 179.26905) (width 0.2) (layer "F.Cu") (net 11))
 (segment (start 119.25 179.26905) (end 119.25 244.25) (width 0.2) (layer "F.Cu") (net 11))
 (segment (start 122.968 247.968) (end 122.968 254.75) (width 0.2) (layer "F.Cu") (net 11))
 (segment (start 119.25 244.25) (end 122.968 247.968) (width 0.2) (layer "F.Cu") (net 11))
 (segment (start 133.76905 237.48095) (end 123.476 247.774) (width 0.2) (layer "F.Cu") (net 10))
 (segment (start 123.476 247.774) (end 123.476 254.75) (width 0.2) (layer "F.Cu") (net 10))
 (segment (start 133.76905 218.75) (end 133.76905 237.48095) (width 0.2) (layer "F.Cu") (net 10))
 (segment (start 123.984 248.266) (end 123.984 254.75) (width 0.2) (layer "F.Cu") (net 9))
 (segment (start 149.25 243.5) (end 147.25 245.5) (width 0.2) (layer "F.Cu") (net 9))
 (segment (start 126.75 245.5) (end 123.984 248.266) (width 0.2) (layer "F.Cu") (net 9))
 (segment (start 149.25 179.26905) (end 149.25 243.5) (width 0.2) (layer "F.Cu") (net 9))
 (segment (start 163.76905 164.75) (end 149.25 179.26905) (width 0.2) (layer "F.Cu") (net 9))
 (segment (start 147.25 245.5) (end 126.75 245.5) (width 0.2) (layer "F.Cu") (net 9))
 (segment (start 163.76905 234.48095) (end 152.25 246) (width 0.2) (layer "F.Cu") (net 8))
 (segment (start 152.25 246) (end 126.9333 246) (width 0.2) (layer "F.Cu") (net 8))
 (segment (start 126.9333 246) (end 124.492 248.4413) (width 0.2) (layer "F.Cu") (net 8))
 (segment (start 163.76905 218.75) (end 163.76905 234.48095) (width 0.2) (layer "F.Cu") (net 8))
 (segment (start 124.492 248.4413) (end 124.492 254.75) (width 0.2) (layer "F.Cu") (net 8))
 (segment (start 123.476 260.274) (end 122.75 261) (width 0.2) (layer "F.Cu") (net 2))
 (segment (start 123.476 258.687) (end 123.476 260.274) (width 0.2) (layer "F.Cu") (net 2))
 (segment (start 125 254.75) (end 125 254.1246) (width 0.2) (layer "F.Cu") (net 3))
 (segment (start 125 254.1246) (end 126.1246 253) (width 0.2) (layer "F.Cu") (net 3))
 (segment (start 126.1246 253) (end 129.5 253) (width 0.2) (layer "F.Cu") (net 3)))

